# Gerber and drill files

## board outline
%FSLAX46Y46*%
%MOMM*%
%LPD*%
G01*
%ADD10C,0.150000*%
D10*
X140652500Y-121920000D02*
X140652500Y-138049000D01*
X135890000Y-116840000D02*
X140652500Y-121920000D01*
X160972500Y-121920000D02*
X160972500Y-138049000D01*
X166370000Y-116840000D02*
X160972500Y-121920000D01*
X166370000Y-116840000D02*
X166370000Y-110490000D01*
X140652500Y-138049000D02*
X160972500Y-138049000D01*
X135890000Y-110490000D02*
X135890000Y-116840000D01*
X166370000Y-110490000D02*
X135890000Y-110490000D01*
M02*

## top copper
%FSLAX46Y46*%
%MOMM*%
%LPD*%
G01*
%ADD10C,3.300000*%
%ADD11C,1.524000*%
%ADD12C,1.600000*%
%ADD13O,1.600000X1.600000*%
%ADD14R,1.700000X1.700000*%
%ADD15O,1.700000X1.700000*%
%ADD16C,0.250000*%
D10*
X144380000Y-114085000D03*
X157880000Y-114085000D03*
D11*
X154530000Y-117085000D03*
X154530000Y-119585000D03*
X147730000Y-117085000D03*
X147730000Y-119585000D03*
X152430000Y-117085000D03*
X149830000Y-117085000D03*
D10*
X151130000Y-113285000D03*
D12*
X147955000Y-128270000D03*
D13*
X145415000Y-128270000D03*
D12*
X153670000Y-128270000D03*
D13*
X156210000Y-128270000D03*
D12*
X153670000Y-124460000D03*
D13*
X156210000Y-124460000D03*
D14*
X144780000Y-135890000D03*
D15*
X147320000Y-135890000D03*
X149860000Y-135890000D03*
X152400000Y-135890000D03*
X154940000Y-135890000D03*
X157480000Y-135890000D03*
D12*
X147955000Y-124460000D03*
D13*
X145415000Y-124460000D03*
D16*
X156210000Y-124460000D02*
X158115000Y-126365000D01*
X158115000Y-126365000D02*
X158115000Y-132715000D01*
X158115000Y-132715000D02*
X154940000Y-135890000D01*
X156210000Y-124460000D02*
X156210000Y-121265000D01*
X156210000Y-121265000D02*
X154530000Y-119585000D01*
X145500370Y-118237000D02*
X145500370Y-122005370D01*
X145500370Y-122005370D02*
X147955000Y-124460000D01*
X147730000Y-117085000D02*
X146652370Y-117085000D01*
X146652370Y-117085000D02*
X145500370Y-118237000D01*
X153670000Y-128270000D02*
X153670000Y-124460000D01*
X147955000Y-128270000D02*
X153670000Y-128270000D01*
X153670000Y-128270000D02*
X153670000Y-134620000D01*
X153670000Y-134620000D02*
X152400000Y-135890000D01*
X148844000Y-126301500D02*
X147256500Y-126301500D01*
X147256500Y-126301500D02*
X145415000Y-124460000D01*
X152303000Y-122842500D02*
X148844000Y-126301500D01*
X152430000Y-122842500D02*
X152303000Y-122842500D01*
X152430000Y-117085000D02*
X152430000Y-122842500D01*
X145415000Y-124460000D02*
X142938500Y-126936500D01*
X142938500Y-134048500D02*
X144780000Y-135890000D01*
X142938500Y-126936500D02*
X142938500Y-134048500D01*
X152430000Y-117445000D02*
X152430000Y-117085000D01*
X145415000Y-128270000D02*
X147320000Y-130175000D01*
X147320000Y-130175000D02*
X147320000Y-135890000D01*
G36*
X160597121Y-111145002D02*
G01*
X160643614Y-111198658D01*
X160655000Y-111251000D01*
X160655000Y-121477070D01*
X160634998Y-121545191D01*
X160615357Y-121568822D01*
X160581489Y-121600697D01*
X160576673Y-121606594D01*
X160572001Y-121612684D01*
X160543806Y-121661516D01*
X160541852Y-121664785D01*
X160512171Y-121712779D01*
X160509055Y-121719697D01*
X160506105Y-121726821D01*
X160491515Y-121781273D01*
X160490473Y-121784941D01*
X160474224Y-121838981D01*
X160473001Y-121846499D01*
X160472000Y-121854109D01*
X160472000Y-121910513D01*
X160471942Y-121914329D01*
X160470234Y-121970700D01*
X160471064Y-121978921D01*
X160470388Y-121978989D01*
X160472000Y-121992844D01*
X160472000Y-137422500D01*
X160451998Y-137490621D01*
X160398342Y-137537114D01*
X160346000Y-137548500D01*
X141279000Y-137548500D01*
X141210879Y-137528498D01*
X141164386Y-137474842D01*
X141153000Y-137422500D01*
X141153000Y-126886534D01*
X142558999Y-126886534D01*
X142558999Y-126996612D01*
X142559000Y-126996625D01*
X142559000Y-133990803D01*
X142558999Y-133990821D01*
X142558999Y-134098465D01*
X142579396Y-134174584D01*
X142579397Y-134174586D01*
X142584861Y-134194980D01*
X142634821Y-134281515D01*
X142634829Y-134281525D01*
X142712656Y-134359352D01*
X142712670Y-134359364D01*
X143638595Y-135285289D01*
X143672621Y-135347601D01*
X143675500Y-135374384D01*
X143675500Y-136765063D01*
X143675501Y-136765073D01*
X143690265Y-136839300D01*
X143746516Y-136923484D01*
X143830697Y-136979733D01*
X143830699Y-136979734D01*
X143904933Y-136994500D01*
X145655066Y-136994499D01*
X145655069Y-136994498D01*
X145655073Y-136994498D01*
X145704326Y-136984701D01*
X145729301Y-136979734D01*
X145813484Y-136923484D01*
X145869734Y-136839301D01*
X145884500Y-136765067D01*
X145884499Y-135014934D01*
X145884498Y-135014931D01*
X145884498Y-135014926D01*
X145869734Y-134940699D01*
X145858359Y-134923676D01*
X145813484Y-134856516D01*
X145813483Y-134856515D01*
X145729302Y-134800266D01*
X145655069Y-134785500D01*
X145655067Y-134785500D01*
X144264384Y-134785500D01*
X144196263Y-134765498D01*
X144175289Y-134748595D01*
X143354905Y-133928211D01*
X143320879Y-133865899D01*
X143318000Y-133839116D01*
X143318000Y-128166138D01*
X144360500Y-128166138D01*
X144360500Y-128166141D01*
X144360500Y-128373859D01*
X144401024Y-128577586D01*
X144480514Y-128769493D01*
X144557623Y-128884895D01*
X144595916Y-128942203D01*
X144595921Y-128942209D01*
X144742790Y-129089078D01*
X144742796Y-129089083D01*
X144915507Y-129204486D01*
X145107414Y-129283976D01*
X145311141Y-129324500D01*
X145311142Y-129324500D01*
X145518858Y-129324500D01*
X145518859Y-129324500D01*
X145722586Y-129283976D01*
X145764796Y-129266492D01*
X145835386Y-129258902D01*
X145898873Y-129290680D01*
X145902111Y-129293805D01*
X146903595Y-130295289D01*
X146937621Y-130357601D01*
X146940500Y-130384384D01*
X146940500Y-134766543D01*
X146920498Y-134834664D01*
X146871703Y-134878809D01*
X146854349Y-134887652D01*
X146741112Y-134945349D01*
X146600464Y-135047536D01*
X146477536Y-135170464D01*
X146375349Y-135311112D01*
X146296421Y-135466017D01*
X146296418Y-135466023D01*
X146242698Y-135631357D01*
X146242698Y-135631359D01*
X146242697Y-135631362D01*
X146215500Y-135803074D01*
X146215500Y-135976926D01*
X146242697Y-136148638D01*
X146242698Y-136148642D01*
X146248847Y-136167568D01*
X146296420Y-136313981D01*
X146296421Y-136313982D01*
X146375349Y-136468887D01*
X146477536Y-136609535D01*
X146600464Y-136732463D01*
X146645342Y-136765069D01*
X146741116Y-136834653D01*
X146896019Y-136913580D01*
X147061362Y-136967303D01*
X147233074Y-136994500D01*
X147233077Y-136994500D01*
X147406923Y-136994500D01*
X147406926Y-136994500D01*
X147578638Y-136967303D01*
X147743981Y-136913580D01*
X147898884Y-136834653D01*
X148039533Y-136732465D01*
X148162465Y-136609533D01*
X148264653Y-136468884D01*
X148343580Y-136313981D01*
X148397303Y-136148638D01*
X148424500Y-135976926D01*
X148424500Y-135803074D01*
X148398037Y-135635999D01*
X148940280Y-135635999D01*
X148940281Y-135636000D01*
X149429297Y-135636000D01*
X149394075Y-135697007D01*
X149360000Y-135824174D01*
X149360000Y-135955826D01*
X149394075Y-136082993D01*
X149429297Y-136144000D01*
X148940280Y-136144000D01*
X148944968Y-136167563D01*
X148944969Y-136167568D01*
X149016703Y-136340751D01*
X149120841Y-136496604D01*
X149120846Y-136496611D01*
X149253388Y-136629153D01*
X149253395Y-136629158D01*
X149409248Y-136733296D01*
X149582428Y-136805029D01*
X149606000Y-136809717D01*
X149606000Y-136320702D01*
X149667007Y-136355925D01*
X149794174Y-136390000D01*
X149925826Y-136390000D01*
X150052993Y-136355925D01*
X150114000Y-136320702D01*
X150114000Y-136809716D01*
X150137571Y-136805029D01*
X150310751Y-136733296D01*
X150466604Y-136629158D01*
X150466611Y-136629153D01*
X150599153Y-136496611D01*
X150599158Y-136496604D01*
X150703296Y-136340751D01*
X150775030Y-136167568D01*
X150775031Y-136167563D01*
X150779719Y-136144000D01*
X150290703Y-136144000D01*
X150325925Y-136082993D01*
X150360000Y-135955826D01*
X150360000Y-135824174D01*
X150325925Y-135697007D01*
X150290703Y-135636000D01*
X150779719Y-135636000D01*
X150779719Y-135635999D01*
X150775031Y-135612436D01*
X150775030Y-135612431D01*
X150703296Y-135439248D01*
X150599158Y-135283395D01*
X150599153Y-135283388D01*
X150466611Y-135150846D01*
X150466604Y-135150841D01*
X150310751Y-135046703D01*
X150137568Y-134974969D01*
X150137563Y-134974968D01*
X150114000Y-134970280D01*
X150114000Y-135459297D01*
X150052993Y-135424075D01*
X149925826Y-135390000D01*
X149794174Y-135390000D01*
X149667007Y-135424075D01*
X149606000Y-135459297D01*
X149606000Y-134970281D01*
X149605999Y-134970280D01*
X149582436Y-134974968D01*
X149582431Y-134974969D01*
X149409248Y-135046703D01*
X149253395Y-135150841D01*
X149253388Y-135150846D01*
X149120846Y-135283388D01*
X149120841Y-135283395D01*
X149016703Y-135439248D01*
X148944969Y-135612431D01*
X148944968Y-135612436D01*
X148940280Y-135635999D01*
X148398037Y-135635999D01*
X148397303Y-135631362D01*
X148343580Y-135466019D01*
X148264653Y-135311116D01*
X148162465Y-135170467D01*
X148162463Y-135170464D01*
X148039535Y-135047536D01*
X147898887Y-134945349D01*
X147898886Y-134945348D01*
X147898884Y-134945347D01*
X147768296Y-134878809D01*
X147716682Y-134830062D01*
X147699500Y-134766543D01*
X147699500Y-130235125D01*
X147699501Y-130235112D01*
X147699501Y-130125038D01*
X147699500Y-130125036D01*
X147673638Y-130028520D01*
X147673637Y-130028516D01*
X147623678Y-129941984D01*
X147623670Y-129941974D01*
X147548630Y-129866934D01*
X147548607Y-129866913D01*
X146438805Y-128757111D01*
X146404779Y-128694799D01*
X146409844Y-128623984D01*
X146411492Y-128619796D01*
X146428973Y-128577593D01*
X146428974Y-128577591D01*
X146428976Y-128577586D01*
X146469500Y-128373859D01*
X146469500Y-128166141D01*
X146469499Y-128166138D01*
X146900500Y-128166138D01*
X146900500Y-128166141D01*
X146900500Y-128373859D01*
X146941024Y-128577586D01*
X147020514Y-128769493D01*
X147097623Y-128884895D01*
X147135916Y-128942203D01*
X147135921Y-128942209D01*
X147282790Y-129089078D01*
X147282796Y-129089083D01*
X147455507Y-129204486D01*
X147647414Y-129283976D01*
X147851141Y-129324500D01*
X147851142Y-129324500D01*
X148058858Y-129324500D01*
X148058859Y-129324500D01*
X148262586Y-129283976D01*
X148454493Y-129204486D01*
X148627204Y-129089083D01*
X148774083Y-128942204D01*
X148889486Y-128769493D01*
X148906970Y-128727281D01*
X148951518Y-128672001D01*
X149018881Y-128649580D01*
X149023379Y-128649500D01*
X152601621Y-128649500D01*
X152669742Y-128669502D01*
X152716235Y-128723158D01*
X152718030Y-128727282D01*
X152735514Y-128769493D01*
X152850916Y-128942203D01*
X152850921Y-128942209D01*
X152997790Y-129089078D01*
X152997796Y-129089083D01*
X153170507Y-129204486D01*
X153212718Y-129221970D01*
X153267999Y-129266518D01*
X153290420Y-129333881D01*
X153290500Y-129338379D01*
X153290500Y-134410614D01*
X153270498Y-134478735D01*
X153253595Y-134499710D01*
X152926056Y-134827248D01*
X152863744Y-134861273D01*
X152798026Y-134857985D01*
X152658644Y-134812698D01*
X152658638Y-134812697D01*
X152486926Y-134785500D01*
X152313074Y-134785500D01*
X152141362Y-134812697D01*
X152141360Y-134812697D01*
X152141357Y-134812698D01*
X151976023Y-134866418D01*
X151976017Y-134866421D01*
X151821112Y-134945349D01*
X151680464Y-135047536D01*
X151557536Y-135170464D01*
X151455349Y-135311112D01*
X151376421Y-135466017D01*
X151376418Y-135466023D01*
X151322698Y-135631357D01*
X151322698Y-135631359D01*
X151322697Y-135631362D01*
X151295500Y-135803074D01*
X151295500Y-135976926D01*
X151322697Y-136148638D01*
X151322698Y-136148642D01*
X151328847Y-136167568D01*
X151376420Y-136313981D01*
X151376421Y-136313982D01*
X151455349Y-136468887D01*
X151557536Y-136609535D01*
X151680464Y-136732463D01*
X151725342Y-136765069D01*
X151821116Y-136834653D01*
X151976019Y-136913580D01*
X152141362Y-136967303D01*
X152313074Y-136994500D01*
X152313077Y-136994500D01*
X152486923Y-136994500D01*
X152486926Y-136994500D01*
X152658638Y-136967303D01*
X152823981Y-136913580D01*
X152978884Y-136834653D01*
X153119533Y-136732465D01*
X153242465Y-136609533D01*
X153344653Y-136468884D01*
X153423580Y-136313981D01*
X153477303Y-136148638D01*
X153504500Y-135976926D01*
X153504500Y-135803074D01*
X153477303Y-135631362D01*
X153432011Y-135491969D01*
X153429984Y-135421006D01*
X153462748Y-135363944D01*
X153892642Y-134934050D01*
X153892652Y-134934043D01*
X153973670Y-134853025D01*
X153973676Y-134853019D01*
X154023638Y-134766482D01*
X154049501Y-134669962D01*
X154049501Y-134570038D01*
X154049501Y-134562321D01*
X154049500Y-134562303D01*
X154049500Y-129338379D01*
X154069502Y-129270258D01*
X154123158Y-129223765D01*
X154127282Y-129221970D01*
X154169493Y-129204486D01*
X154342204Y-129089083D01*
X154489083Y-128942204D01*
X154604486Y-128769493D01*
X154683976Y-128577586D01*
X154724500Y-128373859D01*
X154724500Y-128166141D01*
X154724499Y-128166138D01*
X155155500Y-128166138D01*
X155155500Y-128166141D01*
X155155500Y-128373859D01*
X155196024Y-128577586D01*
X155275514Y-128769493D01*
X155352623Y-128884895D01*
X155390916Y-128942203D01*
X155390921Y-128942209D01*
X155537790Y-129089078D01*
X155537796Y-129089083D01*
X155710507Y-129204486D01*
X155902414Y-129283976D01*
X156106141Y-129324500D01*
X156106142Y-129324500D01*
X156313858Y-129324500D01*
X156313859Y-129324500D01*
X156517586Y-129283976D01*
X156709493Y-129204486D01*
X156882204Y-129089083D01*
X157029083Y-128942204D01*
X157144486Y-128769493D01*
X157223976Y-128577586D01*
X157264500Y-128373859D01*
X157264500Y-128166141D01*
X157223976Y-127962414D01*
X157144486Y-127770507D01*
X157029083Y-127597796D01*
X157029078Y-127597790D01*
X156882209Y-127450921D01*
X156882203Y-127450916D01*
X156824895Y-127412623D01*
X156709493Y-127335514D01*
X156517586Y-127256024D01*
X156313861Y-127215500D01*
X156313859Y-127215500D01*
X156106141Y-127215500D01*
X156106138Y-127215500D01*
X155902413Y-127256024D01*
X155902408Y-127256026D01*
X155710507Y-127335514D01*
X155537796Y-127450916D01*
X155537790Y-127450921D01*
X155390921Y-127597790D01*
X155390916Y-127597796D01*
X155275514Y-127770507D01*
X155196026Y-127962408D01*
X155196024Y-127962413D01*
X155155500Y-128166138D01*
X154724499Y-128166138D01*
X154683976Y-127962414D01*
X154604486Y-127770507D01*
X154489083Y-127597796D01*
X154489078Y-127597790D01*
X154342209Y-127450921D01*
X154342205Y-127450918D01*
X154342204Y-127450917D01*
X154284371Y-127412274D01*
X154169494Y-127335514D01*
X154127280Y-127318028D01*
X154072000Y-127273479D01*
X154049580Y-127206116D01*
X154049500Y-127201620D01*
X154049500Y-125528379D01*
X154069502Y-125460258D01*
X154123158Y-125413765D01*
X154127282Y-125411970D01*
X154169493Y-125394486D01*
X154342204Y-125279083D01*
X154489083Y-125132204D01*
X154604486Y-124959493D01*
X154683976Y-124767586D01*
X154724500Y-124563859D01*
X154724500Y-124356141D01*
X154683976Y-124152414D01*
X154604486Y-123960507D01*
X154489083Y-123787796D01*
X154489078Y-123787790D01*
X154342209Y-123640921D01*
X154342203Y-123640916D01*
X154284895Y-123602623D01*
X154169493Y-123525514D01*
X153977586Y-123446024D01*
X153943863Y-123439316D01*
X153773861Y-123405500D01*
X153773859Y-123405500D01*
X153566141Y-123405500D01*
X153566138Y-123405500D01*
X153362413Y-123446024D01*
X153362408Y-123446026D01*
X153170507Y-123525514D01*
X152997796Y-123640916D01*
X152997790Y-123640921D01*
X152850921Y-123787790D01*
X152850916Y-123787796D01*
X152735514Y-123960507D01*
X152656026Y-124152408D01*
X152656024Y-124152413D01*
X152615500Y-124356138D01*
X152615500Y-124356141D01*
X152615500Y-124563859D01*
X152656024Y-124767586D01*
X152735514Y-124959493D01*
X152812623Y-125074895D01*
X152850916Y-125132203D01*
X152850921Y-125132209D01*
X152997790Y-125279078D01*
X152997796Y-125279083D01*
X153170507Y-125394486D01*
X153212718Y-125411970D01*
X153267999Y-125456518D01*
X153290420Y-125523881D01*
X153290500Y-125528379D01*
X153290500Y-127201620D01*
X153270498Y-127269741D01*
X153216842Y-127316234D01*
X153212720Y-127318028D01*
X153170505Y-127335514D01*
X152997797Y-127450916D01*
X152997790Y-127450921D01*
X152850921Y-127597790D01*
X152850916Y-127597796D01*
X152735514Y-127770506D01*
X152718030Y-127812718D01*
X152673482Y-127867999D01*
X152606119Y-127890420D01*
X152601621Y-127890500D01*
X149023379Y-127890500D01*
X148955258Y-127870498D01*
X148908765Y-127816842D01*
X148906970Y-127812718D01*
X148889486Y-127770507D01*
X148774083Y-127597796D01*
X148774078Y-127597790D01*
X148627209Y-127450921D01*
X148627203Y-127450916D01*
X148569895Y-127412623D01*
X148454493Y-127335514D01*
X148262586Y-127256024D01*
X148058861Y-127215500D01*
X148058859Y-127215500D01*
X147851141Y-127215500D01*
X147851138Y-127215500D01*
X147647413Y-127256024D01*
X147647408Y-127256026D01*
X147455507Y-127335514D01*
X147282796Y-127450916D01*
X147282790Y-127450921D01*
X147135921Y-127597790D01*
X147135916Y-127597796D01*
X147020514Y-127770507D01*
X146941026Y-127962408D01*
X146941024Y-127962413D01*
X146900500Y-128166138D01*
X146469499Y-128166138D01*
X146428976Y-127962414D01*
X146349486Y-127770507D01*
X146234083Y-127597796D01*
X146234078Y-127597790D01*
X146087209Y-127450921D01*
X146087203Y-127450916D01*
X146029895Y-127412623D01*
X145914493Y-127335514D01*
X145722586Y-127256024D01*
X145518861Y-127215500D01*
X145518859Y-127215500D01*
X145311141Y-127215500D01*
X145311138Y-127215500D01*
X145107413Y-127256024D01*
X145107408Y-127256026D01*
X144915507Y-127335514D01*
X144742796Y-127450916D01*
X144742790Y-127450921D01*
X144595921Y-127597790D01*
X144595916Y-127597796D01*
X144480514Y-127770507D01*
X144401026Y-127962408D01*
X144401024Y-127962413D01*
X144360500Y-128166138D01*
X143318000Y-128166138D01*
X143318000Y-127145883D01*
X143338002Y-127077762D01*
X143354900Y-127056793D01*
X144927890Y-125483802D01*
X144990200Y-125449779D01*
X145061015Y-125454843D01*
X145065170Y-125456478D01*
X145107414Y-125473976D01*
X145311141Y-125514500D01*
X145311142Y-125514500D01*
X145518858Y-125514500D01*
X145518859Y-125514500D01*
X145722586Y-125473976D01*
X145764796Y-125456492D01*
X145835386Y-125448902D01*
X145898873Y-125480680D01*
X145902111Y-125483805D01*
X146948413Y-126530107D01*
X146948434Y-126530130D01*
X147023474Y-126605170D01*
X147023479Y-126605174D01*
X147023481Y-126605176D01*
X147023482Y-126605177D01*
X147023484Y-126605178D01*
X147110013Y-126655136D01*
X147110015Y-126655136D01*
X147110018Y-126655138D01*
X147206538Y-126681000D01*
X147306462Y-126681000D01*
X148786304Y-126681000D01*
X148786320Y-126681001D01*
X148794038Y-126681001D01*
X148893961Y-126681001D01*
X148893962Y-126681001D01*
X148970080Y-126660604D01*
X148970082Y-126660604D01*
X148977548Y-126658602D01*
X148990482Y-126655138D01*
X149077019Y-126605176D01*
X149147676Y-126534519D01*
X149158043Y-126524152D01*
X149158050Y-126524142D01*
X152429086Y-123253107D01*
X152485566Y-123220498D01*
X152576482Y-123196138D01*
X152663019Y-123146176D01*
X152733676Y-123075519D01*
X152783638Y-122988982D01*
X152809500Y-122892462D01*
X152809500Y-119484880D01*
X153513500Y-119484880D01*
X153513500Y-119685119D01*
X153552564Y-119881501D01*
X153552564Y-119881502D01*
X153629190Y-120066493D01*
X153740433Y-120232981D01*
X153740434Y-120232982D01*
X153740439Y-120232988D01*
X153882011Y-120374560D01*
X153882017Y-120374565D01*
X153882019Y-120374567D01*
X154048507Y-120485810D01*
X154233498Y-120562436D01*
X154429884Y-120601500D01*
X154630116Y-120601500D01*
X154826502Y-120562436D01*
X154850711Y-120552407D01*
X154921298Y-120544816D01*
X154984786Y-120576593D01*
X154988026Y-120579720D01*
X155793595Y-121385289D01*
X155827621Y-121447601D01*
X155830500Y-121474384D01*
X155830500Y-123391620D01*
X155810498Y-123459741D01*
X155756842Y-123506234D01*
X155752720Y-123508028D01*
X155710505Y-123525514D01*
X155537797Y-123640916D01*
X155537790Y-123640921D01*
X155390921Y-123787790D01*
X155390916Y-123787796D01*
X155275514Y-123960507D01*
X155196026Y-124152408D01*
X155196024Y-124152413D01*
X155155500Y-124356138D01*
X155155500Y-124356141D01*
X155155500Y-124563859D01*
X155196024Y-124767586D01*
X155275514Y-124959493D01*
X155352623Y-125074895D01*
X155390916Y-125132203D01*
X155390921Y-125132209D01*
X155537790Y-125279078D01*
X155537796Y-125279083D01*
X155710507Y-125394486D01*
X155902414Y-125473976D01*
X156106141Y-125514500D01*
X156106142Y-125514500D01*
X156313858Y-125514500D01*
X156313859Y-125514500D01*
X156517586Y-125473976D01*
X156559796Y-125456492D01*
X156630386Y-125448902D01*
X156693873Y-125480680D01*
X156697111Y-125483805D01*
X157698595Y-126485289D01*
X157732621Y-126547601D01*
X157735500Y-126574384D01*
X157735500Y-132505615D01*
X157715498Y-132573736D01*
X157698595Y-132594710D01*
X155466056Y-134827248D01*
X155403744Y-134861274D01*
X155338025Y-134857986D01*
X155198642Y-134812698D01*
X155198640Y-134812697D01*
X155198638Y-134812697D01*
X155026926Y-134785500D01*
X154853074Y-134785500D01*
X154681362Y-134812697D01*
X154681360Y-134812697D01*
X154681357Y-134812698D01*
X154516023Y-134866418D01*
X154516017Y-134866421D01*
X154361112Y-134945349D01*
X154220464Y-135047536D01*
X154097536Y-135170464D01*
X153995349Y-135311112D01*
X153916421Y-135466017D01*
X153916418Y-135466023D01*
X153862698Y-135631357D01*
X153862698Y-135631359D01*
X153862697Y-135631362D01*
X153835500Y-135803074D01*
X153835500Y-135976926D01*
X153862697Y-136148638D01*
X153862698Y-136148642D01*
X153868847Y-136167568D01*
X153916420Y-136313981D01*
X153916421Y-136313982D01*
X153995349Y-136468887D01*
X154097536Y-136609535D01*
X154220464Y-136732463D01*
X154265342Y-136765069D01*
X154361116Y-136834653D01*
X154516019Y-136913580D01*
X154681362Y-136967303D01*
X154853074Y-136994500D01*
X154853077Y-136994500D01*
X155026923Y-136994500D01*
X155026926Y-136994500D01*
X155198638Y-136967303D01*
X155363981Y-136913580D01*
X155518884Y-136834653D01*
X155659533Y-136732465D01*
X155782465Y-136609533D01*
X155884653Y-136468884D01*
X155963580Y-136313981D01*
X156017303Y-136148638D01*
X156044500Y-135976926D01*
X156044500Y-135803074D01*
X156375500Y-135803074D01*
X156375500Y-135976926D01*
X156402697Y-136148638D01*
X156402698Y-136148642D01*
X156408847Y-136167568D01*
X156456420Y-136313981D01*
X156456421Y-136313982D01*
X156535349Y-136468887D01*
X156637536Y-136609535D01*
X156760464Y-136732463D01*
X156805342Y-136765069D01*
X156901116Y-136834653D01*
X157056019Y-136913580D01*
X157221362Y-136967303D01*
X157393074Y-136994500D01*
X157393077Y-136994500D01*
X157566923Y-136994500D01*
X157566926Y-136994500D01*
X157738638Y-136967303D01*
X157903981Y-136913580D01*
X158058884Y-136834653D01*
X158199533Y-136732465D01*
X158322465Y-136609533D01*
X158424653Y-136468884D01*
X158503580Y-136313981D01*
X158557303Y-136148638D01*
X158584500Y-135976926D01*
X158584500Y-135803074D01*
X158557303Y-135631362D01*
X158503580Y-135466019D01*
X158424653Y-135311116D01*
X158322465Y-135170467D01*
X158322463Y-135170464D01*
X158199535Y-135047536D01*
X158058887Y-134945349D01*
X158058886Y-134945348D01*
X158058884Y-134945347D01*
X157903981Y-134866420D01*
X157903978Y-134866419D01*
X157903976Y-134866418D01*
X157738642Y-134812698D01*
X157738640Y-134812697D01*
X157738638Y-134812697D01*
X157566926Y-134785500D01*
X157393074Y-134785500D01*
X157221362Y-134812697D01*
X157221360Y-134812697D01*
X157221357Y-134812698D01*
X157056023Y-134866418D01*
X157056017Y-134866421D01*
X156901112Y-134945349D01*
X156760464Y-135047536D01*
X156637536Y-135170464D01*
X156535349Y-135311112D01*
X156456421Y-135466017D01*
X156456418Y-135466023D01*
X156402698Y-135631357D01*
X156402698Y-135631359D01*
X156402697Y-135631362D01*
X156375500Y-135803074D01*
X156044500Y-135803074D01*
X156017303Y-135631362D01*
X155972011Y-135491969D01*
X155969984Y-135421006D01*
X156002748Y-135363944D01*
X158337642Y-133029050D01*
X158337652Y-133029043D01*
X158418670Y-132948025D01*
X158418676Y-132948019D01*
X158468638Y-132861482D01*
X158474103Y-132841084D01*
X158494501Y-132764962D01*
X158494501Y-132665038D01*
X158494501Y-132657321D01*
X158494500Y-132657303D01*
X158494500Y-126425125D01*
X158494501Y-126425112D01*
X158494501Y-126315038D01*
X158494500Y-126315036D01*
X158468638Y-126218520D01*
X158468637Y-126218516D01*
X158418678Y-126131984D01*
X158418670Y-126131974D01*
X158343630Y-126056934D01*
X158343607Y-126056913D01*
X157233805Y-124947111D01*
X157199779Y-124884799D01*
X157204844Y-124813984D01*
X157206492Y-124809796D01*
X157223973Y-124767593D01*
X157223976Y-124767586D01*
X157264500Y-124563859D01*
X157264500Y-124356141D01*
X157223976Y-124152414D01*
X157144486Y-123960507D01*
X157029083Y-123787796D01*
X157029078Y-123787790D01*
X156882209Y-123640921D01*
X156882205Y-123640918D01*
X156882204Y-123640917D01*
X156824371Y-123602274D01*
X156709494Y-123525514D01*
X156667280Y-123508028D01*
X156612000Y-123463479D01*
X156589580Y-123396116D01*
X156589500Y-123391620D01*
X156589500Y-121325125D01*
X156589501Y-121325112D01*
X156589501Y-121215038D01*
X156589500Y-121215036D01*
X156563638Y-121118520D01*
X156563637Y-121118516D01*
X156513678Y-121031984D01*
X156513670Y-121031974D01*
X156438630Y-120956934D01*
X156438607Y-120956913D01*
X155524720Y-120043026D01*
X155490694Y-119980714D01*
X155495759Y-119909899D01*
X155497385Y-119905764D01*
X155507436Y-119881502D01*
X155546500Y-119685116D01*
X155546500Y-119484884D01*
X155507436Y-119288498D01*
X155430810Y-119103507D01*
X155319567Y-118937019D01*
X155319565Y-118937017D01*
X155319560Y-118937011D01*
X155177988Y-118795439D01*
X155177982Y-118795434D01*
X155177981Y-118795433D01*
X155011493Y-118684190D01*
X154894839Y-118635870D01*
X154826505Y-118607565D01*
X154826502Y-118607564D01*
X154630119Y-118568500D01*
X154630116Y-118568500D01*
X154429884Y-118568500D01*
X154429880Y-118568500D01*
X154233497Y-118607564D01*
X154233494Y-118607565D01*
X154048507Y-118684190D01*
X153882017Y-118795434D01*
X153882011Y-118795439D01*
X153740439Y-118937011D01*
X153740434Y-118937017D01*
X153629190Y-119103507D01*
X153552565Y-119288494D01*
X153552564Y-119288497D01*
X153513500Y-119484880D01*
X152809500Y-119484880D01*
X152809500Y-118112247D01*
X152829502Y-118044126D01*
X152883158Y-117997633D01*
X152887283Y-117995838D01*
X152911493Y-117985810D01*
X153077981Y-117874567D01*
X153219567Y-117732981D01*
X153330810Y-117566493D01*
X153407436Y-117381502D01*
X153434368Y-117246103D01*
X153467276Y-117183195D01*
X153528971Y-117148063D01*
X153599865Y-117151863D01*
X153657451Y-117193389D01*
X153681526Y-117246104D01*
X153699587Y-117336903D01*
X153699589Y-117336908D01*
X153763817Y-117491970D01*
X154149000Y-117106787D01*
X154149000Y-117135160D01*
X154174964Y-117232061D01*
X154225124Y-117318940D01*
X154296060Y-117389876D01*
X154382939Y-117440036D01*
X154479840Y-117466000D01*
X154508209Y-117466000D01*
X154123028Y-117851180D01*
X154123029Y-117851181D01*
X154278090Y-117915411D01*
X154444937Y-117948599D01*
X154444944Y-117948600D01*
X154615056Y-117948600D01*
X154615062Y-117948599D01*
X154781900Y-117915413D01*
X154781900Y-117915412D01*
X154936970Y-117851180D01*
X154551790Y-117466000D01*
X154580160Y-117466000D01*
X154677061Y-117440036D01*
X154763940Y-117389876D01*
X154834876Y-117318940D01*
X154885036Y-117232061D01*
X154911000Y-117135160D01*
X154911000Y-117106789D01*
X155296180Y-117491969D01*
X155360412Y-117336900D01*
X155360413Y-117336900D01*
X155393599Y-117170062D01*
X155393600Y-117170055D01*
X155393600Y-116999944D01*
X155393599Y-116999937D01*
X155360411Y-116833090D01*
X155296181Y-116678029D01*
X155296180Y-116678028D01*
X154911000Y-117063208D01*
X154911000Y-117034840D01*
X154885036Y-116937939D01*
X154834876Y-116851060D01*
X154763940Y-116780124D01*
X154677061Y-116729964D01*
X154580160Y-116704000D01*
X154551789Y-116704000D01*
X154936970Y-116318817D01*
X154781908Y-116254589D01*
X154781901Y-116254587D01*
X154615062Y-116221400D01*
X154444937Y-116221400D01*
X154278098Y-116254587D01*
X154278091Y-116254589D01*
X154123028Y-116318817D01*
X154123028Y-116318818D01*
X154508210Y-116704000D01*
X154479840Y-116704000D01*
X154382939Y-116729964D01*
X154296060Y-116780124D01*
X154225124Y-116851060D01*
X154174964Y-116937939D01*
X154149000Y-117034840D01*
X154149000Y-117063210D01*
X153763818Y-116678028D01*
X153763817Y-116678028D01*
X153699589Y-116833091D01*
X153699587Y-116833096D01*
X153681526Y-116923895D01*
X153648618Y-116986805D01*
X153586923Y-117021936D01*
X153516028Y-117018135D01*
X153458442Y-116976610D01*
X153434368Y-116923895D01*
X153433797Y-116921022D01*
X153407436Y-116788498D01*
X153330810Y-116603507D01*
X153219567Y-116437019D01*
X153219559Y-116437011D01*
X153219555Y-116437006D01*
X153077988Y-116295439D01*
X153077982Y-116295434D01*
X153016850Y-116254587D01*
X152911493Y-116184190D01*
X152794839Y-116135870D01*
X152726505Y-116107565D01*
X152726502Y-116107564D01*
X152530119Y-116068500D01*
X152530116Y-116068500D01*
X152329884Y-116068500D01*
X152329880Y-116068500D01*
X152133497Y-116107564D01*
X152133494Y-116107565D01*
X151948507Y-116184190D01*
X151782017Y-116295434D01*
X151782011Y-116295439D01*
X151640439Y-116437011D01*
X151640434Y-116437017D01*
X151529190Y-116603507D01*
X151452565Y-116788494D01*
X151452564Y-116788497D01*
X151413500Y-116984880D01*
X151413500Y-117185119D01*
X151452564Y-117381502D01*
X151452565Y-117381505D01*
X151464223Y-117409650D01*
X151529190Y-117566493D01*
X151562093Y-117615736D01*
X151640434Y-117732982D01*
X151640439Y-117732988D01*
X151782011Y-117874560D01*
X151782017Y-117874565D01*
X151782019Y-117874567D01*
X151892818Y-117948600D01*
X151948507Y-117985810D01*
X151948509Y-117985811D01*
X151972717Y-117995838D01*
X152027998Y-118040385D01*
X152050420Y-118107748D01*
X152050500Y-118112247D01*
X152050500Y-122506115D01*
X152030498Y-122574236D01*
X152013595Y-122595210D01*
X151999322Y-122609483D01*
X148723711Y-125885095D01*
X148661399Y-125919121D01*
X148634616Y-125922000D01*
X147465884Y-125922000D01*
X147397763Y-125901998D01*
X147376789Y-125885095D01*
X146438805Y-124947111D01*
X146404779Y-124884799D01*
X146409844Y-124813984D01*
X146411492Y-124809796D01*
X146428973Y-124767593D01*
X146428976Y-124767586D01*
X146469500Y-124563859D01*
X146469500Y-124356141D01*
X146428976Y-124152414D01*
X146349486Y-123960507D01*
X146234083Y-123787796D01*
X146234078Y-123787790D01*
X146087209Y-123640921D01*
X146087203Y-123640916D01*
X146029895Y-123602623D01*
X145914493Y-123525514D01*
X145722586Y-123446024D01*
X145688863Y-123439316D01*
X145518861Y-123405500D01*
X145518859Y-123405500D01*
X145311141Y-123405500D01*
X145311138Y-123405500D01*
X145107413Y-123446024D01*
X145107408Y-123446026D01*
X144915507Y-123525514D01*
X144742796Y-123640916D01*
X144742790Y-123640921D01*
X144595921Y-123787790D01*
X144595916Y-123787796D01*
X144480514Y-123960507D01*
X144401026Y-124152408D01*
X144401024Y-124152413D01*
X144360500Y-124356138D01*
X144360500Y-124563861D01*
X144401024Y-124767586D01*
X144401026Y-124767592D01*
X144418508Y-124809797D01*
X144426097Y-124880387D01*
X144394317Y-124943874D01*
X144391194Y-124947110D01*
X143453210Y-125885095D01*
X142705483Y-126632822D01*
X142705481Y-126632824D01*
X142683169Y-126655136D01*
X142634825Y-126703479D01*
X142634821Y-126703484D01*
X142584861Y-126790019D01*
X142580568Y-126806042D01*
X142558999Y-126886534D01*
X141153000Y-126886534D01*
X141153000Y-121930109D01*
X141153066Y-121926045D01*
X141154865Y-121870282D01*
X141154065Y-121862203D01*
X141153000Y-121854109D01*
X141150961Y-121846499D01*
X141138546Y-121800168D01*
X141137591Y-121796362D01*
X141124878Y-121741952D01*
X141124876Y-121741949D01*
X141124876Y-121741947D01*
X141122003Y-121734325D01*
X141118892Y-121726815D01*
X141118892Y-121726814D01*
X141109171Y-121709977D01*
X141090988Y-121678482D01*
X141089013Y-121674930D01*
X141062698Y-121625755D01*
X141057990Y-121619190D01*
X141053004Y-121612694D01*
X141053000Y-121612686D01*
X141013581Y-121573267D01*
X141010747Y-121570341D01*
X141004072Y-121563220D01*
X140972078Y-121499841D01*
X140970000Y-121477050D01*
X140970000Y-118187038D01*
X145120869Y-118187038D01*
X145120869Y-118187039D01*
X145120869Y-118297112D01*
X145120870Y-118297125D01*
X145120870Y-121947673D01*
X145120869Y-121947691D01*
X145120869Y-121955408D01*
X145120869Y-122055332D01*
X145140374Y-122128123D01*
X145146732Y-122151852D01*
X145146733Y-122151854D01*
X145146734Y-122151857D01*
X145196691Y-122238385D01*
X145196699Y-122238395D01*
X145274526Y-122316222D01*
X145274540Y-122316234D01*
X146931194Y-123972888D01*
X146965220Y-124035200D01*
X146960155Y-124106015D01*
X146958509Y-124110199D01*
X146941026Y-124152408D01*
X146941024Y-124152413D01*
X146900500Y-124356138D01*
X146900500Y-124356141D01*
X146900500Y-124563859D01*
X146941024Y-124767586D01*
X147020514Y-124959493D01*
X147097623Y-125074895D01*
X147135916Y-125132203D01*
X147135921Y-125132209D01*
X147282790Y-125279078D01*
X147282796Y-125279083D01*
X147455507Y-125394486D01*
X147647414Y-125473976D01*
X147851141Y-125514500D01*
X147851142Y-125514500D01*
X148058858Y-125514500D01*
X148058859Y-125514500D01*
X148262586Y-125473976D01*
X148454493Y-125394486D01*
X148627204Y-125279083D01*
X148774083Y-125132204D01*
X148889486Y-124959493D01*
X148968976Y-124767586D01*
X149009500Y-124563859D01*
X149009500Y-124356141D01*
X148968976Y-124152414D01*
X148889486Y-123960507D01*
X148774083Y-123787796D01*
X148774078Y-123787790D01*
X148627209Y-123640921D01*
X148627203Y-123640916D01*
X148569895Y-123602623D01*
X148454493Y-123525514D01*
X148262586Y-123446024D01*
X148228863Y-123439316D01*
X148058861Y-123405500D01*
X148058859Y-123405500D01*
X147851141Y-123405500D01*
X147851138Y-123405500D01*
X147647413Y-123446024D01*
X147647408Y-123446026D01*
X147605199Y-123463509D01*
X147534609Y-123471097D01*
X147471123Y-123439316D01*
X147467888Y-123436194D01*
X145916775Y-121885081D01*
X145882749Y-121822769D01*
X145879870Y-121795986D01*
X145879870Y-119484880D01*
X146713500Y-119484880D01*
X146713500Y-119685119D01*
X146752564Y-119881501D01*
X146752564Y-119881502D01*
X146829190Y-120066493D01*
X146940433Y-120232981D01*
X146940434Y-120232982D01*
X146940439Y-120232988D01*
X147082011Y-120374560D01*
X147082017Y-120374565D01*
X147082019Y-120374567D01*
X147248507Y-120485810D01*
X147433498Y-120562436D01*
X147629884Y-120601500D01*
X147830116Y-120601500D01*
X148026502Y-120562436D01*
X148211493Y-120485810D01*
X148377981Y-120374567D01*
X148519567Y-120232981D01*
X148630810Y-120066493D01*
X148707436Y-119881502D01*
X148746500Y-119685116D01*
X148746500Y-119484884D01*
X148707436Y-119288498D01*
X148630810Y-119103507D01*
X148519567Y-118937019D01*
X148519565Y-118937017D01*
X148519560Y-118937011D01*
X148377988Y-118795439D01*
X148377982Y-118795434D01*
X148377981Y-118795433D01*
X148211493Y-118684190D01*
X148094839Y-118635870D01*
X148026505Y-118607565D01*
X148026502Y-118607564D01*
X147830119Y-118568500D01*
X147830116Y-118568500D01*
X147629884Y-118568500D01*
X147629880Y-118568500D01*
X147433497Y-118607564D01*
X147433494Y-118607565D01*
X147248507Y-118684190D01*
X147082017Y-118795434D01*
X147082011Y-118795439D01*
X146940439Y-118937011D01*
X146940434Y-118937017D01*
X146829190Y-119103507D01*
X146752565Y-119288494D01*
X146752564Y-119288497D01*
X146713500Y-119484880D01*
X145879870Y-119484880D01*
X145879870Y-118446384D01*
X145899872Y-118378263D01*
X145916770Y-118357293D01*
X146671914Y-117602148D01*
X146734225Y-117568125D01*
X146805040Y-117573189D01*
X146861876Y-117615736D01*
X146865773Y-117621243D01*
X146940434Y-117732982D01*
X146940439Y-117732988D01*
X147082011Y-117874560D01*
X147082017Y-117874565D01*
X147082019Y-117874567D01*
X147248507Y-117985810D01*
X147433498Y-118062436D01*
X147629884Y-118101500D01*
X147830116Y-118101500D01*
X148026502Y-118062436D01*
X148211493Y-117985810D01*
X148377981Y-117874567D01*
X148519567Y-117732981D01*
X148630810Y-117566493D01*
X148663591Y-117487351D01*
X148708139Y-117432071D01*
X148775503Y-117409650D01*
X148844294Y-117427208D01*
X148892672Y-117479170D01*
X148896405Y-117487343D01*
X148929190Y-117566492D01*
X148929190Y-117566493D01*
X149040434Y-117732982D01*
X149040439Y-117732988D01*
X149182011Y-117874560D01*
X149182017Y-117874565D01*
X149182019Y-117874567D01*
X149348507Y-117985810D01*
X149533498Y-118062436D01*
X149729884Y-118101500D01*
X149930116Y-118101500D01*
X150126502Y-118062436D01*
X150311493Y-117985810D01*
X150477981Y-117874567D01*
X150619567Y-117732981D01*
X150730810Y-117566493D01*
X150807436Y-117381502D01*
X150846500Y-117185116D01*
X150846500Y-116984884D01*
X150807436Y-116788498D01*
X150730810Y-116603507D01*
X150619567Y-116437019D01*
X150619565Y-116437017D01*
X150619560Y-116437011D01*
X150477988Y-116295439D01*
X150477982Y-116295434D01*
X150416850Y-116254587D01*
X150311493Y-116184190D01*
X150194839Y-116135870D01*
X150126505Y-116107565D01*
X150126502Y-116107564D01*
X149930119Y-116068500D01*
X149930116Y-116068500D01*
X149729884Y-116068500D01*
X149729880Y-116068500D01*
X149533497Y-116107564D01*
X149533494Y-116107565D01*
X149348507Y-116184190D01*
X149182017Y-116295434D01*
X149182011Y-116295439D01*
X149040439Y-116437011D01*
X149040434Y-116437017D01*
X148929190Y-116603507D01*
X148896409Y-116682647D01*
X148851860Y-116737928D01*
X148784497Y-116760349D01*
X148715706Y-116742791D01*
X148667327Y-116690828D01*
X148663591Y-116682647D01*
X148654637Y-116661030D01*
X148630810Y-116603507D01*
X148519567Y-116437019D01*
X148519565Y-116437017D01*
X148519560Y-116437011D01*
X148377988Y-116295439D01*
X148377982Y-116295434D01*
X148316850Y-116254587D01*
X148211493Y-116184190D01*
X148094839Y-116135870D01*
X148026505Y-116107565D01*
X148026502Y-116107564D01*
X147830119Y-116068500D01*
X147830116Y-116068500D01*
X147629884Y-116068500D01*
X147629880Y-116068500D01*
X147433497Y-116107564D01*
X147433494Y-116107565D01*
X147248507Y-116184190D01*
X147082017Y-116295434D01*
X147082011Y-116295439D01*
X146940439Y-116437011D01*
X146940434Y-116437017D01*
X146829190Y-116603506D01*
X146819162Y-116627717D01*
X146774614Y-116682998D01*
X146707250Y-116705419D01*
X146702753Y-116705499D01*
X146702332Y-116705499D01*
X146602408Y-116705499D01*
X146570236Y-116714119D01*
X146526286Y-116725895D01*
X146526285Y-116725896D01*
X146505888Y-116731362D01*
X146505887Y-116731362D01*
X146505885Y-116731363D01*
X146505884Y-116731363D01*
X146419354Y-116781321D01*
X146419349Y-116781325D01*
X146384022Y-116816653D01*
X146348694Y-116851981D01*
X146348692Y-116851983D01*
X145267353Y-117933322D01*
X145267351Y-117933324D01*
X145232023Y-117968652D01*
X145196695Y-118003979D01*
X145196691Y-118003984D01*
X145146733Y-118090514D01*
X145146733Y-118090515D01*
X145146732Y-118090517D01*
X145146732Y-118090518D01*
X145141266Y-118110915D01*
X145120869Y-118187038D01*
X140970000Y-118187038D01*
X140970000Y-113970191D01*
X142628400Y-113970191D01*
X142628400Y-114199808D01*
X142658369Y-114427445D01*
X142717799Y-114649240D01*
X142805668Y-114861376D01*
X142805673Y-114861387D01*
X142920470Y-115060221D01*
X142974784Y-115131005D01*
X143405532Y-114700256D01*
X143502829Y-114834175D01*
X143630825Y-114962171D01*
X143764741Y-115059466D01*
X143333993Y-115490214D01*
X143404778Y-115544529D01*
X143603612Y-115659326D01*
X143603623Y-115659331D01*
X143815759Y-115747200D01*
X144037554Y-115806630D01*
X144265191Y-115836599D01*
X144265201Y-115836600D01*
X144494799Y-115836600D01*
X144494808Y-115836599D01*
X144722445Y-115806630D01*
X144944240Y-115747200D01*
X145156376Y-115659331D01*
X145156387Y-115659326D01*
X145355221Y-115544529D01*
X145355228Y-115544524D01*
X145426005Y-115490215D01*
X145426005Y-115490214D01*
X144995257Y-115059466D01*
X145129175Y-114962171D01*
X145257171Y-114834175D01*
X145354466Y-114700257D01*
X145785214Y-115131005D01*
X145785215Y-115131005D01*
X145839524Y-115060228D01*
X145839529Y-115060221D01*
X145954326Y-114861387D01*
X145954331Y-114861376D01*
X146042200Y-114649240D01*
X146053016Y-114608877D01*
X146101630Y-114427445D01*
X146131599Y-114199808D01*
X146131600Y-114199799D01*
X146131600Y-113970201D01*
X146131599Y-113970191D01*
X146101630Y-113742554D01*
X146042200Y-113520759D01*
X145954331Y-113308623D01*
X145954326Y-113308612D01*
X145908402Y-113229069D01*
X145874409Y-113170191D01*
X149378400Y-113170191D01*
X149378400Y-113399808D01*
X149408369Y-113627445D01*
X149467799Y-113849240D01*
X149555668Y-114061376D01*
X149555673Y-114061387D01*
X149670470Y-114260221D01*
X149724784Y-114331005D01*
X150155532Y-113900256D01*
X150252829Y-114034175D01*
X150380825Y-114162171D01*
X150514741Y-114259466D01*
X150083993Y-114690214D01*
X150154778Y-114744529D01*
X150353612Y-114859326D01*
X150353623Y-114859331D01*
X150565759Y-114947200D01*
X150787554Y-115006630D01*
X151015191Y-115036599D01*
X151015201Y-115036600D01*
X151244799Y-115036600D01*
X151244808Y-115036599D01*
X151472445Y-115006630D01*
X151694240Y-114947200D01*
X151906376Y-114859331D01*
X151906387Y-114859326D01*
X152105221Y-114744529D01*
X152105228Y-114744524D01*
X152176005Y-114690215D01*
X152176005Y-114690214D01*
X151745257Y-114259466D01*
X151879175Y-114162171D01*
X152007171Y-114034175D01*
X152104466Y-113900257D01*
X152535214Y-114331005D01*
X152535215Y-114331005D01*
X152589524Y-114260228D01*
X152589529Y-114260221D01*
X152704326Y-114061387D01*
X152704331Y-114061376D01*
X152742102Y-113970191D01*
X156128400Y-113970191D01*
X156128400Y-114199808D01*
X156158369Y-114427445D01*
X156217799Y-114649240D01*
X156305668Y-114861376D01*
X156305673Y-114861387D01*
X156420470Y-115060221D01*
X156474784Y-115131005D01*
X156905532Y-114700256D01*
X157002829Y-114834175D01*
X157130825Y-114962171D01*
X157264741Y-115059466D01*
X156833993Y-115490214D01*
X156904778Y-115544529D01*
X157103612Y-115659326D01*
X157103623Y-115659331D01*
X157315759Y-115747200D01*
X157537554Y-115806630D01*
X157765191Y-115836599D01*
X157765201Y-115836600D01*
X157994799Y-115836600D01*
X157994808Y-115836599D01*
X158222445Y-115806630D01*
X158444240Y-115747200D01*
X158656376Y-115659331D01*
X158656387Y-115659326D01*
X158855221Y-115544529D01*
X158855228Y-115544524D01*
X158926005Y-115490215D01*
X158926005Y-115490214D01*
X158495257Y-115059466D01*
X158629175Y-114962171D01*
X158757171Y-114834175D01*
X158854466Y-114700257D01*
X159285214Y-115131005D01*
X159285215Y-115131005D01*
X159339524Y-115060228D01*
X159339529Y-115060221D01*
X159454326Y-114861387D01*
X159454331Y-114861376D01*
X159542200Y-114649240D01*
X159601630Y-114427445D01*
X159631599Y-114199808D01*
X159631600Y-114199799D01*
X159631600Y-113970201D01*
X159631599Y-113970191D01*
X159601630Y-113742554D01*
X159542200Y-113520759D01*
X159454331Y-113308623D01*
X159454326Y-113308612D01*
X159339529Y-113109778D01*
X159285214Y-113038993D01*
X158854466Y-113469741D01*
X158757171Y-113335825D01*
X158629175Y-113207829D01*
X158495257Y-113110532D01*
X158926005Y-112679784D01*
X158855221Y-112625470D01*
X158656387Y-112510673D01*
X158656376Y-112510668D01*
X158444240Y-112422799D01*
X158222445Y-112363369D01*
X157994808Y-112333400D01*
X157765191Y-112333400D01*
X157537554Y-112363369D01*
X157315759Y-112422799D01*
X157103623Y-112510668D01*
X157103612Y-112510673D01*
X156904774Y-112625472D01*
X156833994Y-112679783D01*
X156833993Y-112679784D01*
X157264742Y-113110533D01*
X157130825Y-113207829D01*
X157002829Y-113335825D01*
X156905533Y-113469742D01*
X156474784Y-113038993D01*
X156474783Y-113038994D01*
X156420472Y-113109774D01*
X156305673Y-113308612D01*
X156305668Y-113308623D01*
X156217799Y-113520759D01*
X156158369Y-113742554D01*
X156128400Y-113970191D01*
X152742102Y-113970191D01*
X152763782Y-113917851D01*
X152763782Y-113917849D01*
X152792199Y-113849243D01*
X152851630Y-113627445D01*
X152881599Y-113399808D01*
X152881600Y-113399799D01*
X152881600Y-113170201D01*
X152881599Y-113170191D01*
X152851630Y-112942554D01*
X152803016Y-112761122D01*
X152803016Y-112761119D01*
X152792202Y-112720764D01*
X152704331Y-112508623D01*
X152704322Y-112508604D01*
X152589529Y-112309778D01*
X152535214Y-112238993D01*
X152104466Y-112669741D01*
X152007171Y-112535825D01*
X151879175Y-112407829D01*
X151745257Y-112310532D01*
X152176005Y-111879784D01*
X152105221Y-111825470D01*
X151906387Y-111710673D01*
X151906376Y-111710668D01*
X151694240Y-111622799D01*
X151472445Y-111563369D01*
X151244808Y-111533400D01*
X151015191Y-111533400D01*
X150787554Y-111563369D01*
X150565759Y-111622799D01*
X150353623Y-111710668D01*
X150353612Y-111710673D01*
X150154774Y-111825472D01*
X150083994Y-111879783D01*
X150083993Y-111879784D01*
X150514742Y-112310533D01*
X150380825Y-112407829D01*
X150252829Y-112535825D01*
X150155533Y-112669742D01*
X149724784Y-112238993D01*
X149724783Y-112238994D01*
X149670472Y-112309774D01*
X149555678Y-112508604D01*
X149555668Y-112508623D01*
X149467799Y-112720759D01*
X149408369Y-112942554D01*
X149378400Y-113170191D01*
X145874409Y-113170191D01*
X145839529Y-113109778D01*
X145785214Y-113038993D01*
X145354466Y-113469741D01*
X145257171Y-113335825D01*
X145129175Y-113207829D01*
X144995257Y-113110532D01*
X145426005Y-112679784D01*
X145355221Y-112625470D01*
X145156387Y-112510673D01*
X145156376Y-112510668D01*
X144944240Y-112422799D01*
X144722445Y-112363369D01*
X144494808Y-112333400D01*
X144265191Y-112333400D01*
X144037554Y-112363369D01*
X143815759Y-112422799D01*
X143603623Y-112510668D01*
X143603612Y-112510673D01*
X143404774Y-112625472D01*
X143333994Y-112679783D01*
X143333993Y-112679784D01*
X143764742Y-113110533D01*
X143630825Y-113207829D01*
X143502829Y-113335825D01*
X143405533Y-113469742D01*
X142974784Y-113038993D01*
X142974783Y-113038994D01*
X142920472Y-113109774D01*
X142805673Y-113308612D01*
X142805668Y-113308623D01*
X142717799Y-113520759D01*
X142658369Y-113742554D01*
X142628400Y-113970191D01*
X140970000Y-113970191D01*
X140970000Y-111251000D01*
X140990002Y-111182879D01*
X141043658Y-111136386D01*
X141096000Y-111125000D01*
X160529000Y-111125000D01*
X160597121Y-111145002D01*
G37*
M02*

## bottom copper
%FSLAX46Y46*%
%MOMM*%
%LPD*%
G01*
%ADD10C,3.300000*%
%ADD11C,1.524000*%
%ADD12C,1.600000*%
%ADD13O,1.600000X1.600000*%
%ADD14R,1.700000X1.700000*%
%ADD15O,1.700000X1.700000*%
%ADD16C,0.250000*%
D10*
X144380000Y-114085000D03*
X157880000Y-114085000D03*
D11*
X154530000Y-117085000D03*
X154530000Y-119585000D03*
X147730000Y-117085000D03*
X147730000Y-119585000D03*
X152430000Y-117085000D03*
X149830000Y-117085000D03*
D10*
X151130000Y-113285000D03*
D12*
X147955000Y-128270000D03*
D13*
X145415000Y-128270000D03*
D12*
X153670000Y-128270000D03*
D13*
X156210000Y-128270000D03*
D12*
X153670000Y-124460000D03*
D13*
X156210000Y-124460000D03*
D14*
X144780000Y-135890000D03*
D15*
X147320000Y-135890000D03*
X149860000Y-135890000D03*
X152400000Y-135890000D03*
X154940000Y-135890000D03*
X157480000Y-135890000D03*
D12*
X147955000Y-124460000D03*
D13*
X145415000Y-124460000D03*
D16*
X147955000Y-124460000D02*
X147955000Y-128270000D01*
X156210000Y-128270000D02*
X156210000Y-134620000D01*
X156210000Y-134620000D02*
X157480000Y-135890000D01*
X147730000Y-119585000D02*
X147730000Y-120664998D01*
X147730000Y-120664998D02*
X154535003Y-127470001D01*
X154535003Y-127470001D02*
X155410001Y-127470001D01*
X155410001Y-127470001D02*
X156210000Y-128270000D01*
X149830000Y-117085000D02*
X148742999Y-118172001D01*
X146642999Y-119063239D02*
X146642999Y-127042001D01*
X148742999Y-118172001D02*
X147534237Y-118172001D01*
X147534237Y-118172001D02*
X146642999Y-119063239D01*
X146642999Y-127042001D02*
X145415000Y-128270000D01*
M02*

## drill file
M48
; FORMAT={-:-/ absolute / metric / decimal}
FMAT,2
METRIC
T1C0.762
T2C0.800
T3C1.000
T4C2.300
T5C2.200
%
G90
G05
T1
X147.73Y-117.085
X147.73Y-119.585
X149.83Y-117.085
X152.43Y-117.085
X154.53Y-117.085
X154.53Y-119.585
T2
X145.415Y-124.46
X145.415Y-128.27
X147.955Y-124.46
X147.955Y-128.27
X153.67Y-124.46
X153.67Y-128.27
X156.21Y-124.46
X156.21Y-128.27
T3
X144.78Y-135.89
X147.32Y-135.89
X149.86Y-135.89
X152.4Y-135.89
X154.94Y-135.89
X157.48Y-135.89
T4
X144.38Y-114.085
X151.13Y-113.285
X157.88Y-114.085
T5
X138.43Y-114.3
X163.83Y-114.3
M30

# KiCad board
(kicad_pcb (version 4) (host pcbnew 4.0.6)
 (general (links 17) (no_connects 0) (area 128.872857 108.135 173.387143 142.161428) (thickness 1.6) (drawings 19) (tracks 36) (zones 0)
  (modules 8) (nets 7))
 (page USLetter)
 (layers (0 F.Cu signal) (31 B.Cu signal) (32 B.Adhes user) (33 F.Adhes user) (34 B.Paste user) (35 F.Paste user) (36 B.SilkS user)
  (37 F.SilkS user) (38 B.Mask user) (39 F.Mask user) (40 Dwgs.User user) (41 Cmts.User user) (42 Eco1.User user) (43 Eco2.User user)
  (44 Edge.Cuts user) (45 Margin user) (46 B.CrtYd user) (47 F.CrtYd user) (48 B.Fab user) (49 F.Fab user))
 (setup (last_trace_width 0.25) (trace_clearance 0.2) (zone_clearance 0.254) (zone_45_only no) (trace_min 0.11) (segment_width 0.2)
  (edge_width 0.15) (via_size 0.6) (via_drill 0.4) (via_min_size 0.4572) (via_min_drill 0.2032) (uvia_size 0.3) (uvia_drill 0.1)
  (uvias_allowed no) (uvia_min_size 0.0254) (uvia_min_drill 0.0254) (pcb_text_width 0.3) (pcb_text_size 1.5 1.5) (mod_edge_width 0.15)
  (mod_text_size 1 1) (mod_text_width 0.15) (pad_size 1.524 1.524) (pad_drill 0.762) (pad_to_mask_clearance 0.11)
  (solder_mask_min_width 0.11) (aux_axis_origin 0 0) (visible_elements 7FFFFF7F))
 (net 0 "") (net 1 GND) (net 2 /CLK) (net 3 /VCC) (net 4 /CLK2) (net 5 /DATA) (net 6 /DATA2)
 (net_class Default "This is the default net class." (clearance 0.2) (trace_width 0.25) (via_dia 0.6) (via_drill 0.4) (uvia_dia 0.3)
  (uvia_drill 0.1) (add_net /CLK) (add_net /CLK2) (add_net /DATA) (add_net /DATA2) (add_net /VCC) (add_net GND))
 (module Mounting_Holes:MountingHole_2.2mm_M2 (layer F.Cu) (at 163.83 114.3)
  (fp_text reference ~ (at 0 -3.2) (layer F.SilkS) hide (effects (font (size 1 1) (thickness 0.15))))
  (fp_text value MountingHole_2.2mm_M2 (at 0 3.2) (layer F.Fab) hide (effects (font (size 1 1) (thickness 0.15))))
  (pad 1 np_thru_hole circle (at 0 0) (size 2.2 2.2) (drill 2.2) (layers *.Cu *.Mask)))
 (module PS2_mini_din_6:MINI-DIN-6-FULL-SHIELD (layer F.Cu) (at 151.13 108.585)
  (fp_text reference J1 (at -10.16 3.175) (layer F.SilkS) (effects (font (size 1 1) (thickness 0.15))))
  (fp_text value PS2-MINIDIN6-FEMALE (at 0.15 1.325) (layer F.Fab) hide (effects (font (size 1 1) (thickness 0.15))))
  (pad 7 thru_hole circle (at -6.75 5.5) (size 3.3 3.3) (drill 2.3) (layers *.Cu *.Mask) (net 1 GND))
  (pad 7 thru_hole circle (at 6.75 5.5) (size 3.3 3.3) (drill 2.3) (layers *.Cu *.Mask) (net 1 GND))
  (pad 3 thru_hole circle (at 3.4 8.5) (size 1.524 1.524) (drill 0.762) (layers *.Cu *.Mask) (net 1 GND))
  (pad 5 thru_hole circle (at 3.4 11) (size 1.524 1.524) (drill 0.762) (layers *.Cu *.Mask) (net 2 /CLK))
  (pad 4 thru_hole circle (at -3.4 8.5) (size 1.524 1.524) (drill 0.762) (layers *.Cu *.Mask) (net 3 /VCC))
  (pad 6 thru_hole circle (at -3.4 11) (size 1.524 1.524) (drill 0.762) (layers *.Cu *.Mask) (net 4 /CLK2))
  (pad 1 thru_hole circle (at 1.3 8.5) (size 1.524 1.524) (drill 0.762) (layers *.Cu *.Mask) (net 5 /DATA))
  (pad 2 thru_hole circle (at -1.3 8.5) (size 1.524 1.524) (drill 0.762) (layers *.Cu *.Mask) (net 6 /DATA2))
  (pad 7 thru_hole circle (at 0 4.7) (size 3.3 3.3) (drill 2.3) (layers *.Cu *.Mask) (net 1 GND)))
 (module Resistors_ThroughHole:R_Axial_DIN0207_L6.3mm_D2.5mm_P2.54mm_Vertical (layer F.Cu) (at 147.955 128.27 180)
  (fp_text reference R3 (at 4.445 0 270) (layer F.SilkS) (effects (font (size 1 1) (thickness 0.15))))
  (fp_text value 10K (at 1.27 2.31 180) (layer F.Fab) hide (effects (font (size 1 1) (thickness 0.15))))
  (pad 1 thru_hole circle (at 0 0 180) (size 1.6 1.6) (drill 0.8) (layers *.Cu *.Mask) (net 3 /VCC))
  (pad 2 thru_hole oval (at 2.54 0 180) (size 1.6 1.6) (drill 0.8) (layers *.Cu *.Mask) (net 6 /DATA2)))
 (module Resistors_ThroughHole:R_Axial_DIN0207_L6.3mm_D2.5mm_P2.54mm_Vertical (layer F.Cu) (at 153.67 128.27)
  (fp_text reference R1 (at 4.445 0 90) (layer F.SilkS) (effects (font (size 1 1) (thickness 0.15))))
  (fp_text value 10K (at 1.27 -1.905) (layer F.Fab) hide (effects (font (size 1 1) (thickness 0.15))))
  (pad 1 thru_hole circle (at 0 0) (size 1.6 1.6) (drill 0.8) (layers *.Cu *.Mask) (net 3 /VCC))
  (pad 2 thru_hole oval (at 2.54 0) (size 1.6 1.6) (drill 0.8) (layers *.Cu *.Mask) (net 4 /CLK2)))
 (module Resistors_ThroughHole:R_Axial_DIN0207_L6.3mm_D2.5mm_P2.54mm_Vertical (layer F.Cu) (at 153.67 124.46)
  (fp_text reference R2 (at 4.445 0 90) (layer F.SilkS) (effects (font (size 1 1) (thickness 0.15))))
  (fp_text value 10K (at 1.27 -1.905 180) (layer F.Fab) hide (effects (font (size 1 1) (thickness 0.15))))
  (pad 1 thru_hole circle (at 0 0) (size 1.6 1.6) (drill 0.8) (layers *.Cu *.Mask) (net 3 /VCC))
  (pad 2 thru_hole oval (at 2.54 0) (size 1.6 1.6) (drill 0.8) (layers *.Cu *.Mask) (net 2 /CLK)))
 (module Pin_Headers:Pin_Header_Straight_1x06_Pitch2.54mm (layer F.Cu) (at 144.78 135.89 90)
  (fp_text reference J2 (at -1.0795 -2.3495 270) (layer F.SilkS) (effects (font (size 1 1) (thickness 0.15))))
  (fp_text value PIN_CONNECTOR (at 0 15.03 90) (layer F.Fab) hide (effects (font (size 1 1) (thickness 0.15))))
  (pad 1 thru_hole rect (at 0 0 90) (size 1.7 1.7) (drill 1) (layers *.Cu *.Mask) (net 5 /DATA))
  (pad 2 thru_hole oval (at 0 2.54 90) (size 1.7 1.7) (drill 1) (layers *.Cu *.Mask) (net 6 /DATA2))
  (pad 3 thru_hole oval (at 0 5.08 90) (size 1.7 1.7) (drill 1) (layers *.Cu *.Mask) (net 1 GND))
  (pad 4 thru_hole oval (at 0 7.62 90) (size 1.7 1.7) (drill 1) (layers *.Cu *.Mask) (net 3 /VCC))
  (pad 5 thru_hole oval (at 0 10.16 90) (size 1.7 1.7) (drill 1) (layers *.Cu *.Mask) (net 2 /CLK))
  (pad 6 thru_hole oval (at 0 12.7 90) (size 1.7 1.7) (drill 1) (layers *.Cu *.Mask) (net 4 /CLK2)))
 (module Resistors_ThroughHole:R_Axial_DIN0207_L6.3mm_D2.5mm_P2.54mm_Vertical (layer F.Cu) (at 147.955 124.46 180)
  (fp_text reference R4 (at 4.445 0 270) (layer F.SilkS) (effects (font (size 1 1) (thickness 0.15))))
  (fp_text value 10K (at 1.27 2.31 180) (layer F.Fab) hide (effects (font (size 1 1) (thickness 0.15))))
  (pad 1 thru_hole circle (at 0 0 180) (size 1.6 1.6) (drill 0.8) (layers *.Cu *.Mask) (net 3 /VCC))
  (pad 2 thru_hole oval (at 2.54 0 180) (size 1.6 1.6) (drill 0.8) (layers *.Cu *.Mask) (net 5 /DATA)))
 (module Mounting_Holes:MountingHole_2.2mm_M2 (layer F.Cu) (at 138.43 114.3)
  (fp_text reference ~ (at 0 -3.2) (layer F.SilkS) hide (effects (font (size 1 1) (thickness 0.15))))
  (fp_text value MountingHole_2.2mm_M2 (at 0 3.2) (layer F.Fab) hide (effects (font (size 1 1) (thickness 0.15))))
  (pad 1 np_thru_hole circle (at 0 0) (size 2.2 2.2) (drill 2.2) (layers *.Cu *.Mask)))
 (gr_line (start 140.6525 121.92) (end 140.6525 138.049) (layer Edge.Cuts) (width 0.15))
 (gr_line (start 135.89 116.84) (end 140.6525 121.92) (layer Edge.Cuts) (width 0.15))
 (gr_line (start 160.9725 121.92) (end 160.9725 138.049) (layer Edge.Cuts) (width 0.15))
 (gr_line (start 166.37 116.84) (end 160.9725 121.92) (layer Edge.Cuts) (width 0.15))
 (gr_line (start 166.37 116.84) (end 166.37 110.49) (layer Edge.Cuts) (width 0.15))
 (gr_line (start 140.6525 138.049) (end 160.9725 138.049) (layer Edge.Cuts) (width 0.15))
 (gr_line (start 135.89 110.49) (end 135.89 116.84) (layer Edge.Cuts) (width 0.15))
 (gr_line (start 166.37 110.49) (end 135.89 110.49) (layer Edge.Cuts) (width 0.15))
 (segment (start 156.21 124.46) (end 158.115 126.365) (width 0.25) (layer F.Cu) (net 2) (status 10))
 (segment (start 158.115 126.365) (end 158.115 132.715) (width 0.25) (layer F.Cu) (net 2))
 (segment (start 158.115 132.715) (end 154.94 135.89) (width 0.25) (layer F.Cu) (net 2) (status 20))
 (segment (start 156.21 124.46) (end 156.21 121.265) (width 0.25) (layer F.Cu) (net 2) (status 10))
 (segment (start 156.21 121.265) (end 154.53 119.585) (width 0.25) (layer F.Cu) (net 2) (status 20))
 (segment (start 145.50037 118.237) (end 145.50037 122.00537) (width 0.25) (layer F.Cu) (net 3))
 (segment (start 145.50037 122.00537) (end 147.955 124.46) (width 0.25) (layer F.Cu) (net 3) (status 20))
 (segment (start 147.73 117.085) (end 146.65237 117.085) (width 0.25) (layer F.Cu) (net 3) (status 10))
 (segment (start 146.65237 117.085) (end 145.50037 118.237) (width 0.25) (layer F.Cu) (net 3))
 (segment (start 153.67 128.27) (end 153.67 124.46) (width 0.25) (layer F.Cu) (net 3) (status 30))
 (segment (start 147.955 128.27) (end 153.67 128.27) (width 0.25) (layer F.Cu) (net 3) (status 30))
 (segment (start 153.67 128.27) (end 153.67 134.62) (width 0.25) (layer F.Cu) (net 3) (status 10))
 (segment (start 153.67 134.62) (end 152.4 135.89) (width 0.25) (layer F.Cu) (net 3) (status 20))
 (segment (start 147.955 124.46) (end 147.955 128.27) (width 0.25) (layer B.Cu) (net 3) (status 30))
 (segment (start 156.21 128.27) (end 156.21 134.62) (width 0.25) (layer B.Cu) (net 4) (status 10))
 (segment (start 156.21 134.62) (end 157.48 135.89) (width 0.25) (layer B.Cu) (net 4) (status 20))
 (segment (start 147.73 119.585) (end 147.73 120.664998) (width 0.25) (layer B.Cu) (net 4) (status 10))
 (segment (start 147.73 120.664998) (end 154.535003 127.470001) (width 0.25) (layer B.Cu) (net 4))
 (segment (start 154.535003 127.470001) (end 155.410001 127.470001) (width 0.25) (layer B.Cu) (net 4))
 (segment (start 155.410001 127.470001) (end 156.21 128.27) (width 0.25) (layer B.Cu) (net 4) (status 20))
 (segment (start 148.844 126.3015) (end 147.2565 126.3015) (width 0.25) (layer F.Cu) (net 5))
 (segment (start 147.2565 126.3015) (end 145.415 124.46) (width 0.25) (layer F.Cu) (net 5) (status 20))
 (segment (start 152.303 122.8425) (end 148.844 126.3015) (width 0.25) (layer F.Cu) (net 5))
 (segment (start 152.43 122.8425) (end 152.303 122.8425) (width 0.25) (layer F.Cu) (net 5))
 (segment (start 152.43 117.085) (end 152.43 122.8425) (width 0.25) (layer F.Cu) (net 5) (status 10))
 (segment (start 145.415 124.46) (end 142.9385 126.9365) (width 0.25) (layer F.Cu) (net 5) (status 10))
 (segment (start 142.9385 134.0485) (end 144.78 135.89) (width 0.25) (layer F.Cu) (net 5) (status 20))
 (segment (start 142.9385 126.9365) (end 142.9385 134.0485) (width 0.25) (layer F.Cu) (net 5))
 (segment (start 152.43 117.445) (end 152.43 117.085) (width 0.25) (layer F.Cu) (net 5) (status 30))
 (segment (start 145.415 128.27) (end 147.32 130.175) (width 0.25) (layer F.Cu) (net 6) (status 10))
 (segment (start 147.32 130.175) (end 147.32 135.89) (width 0.25) (layer F.Cu) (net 6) (status 20))
 (segment (start 149.83 117.085) (end 148.742999 118.172001) (width 0.25) (layer B.Cu) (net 6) (status 10))
 (segment (start 146.642999 119.063239) (end 146.642999 127.042001) (width 0.25) (layer B.Cu) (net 6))
 (segment (start 148.742999 118.172001) (end 147.534237 118.172001) (width 0.25) (layer B.Cu) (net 6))
 (segment (start 147.534237 118.172001) (end 146.642999 119.063239) (width 0.25) (layer B.Cu) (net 6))
 (segment (start 146.642999 127.042001) (end 145.415 128.27) (width 0.25) (layer B.Cu) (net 6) (status 20))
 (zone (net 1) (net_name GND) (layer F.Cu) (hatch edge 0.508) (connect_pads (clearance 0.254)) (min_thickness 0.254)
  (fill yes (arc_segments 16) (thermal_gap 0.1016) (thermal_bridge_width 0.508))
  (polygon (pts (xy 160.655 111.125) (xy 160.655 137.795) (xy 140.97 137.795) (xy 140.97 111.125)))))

